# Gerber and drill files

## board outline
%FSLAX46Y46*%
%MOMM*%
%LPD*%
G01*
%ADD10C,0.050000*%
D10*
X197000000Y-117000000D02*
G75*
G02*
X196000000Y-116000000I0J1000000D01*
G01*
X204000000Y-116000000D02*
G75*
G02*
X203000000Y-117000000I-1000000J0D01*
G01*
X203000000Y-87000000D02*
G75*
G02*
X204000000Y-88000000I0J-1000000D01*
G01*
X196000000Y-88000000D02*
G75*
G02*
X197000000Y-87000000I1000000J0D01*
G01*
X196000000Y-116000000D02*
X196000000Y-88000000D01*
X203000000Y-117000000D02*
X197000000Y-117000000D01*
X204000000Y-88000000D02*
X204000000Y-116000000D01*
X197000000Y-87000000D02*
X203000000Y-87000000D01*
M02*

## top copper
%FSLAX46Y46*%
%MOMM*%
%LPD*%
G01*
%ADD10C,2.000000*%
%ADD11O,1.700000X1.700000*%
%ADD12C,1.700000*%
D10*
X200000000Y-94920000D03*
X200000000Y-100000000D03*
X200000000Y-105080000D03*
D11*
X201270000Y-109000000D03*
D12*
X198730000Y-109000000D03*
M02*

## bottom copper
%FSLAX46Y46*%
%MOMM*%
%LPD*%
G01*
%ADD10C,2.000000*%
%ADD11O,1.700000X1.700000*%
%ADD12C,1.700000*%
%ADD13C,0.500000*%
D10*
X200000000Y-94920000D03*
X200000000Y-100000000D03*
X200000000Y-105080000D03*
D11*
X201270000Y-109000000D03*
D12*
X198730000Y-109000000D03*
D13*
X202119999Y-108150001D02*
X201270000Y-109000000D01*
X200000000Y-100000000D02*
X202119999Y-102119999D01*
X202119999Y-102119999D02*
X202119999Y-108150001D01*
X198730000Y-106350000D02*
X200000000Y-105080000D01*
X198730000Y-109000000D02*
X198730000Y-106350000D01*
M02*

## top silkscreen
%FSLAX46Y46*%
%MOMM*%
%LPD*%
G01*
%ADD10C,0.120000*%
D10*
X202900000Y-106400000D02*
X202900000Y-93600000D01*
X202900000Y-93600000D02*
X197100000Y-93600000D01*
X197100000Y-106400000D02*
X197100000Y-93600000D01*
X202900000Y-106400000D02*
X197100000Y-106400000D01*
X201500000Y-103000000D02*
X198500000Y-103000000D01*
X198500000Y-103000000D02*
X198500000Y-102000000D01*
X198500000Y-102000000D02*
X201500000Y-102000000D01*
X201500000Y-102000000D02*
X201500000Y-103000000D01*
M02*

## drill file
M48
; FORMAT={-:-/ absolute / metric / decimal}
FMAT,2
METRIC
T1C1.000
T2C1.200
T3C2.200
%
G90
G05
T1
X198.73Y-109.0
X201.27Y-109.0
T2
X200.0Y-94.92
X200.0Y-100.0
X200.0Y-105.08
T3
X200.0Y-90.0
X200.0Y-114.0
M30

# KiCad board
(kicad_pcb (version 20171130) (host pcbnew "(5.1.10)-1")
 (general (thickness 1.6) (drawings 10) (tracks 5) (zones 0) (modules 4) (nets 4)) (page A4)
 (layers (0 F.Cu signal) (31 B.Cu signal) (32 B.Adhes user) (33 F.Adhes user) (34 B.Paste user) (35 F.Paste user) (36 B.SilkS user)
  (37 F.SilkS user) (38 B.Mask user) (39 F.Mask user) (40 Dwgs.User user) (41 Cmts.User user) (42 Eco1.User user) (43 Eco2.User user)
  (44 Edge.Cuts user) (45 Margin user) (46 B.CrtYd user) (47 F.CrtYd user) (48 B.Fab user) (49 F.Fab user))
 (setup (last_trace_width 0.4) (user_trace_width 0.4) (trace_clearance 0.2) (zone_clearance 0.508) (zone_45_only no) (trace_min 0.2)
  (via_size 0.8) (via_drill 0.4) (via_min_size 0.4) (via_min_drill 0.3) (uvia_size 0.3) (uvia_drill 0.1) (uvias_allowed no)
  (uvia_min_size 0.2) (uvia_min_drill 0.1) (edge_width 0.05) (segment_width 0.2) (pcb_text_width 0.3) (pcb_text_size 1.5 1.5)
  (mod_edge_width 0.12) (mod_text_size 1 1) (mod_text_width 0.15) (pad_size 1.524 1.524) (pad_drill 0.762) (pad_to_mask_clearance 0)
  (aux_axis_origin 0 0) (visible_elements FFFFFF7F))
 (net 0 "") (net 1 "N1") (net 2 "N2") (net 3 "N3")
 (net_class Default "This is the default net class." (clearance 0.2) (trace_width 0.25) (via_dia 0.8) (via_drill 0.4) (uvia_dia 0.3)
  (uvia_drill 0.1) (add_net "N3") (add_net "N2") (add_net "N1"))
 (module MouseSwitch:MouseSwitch (layer F.Cu) (at 200 100 180)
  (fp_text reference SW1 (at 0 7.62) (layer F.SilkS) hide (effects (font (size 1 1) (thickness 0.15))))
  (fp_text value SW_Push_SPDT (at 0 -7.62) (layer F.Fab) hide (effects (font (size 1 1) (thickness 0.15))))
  (fp_line (start -2.9 -6.4) (end -2.9 6.4) (layer F.SilkS) (width 0.12))
  (fp_line (start -2.9 6.4) (end 2.9 6.4) (layer F.SilkS) (width 0.12))
  (fp_line (start 2.9 -6.4) (end 2.9 6.4) (layer F.SilkS) (width 0.12))
  (fp_line (start -2.9 -6.4) (end 2.9 -6.4) (layer F.SilkS) (width 0.12))
  (fp_line (start -1.5 -3) (end 1.5 -3) (layer F.SilkS) (width 0.12))
  (fp_line (start 1.5 -3) (end 1.5 -2) (layer F.SilkS) (width 0.12))
  (fp_line (start 1.5 -2) (end -1.5 -2) (layer F.SilkS) (width 0.12))
  (fp_line (start -1.5 -2) (end -1.5 -3) (layer F.SilkS) (width 0.12))
  (pad 1 thru_hole circle (at 0 5.08 180) (size 2 2) (drill 1.2) (layers *.Cu *.Mask) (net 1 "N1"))
  (pad 3 thru_hole circle (at 0 0 180) (size 2 2) (drill 1.2) (layers *.Cu *.Mask) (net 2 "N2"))
  (pad 2 thru_hole circle (at 0 -5.08 180) (size 2 2) (drill 1.2) (layers *.Cu *.Mask) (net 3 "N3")))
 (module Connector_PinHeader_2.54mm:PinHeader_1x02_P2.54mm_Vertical (layer F.Cu) (at 198.73 109 90)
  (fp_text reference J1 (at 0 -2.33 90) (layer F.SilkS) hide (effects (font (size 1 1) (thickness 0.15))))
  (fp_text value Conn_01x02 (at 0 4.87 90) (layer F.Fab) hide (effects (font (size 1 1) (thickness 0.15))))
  (pad 2 thru_hole oval (at 0 2.54 90) (size 1.7 1.7) (drill 1) (layers *.Cu *.Mask) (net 2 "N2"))
  (pad 1 thru_hole circle (at 0 0 90) (size 1.7 1.7) (drill 1) (layers *.Cu *.Mask) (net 3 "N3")))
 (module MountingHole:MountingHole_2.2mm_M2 (layer F.Cu) (at 200 114)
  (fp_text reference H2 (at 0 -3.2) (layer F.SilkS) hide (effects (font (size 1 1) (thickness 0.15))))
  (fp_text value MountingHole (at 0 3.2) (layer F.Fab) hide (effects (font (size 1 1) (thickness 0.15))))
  (pad 1 np_thru_hole circle (at 0 0) (size 2.2 2.2) (drill 2.2) (layers *.Cu *.Mask)))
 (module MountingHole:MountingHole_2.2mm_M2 (layer F.Cu) (at 200 90)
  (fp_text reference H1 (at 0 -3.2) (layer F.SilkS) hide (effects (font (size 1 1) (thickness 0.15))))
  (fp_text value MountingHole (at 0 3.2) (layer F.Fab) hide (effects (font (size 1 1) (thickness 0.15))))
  (pad 1 np_thru_hole circle (at 0 0) (size 2.2 2.2) (drill 2.2) (layers *.Cu *.Mask)))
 (gr_arc (start 197 116) (end 196 116) (angle -90) (layer Edge.Cuts) (width 0.05))
 (gr_arc (start 203 116) (end 203 117) (angle -90) (layer Edge.Cuts) (width 0.05))
 (gr_arc (start 203 88) (end 204 88) (angle -90) (layer Edge.Cuts) (width 0.05))
 (gr_arc (start 197 88) (end 197 87) (angle -90) (layer Edge.Cuts) (width 0.05))
 (gr_line (start 196 116) (end 196 88) (layer Edge.Cuts) (width 0.05))
 (gr_line (start 203 117) (end 197 117) (layer Edge.Cuts) (width 0.05))
 (gr_line (start 204 88) (end 204 116) (layer Edge.Cuts) (width 0.05))
 (gr_line (start 197 87) (end 203 87) (layer Edge.Cuts) (width 0.05))
 (segment (start 202.119999 108.150001) (end 201.27 109) (width 0.5) (layer B.Cu) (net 2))
 (segment (start 200 100) (end 202.119999 102.119999) (width 0.5) (layer B.Cu) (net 2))
 (segment (start 202.119999 102.119999) (end 202.119999 108.150001) (width 0.5) (layer B.Cu) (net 2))
 (segment (start 198.73 106.35) (end 200 105.08) (width 0.5) (layer B.Cu) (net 3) (status 1000000))
 (segment (start 198.73 109) (end 198.73 106.35) (width 0.5) (layer B.Cu) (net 3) (status 1000000)))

